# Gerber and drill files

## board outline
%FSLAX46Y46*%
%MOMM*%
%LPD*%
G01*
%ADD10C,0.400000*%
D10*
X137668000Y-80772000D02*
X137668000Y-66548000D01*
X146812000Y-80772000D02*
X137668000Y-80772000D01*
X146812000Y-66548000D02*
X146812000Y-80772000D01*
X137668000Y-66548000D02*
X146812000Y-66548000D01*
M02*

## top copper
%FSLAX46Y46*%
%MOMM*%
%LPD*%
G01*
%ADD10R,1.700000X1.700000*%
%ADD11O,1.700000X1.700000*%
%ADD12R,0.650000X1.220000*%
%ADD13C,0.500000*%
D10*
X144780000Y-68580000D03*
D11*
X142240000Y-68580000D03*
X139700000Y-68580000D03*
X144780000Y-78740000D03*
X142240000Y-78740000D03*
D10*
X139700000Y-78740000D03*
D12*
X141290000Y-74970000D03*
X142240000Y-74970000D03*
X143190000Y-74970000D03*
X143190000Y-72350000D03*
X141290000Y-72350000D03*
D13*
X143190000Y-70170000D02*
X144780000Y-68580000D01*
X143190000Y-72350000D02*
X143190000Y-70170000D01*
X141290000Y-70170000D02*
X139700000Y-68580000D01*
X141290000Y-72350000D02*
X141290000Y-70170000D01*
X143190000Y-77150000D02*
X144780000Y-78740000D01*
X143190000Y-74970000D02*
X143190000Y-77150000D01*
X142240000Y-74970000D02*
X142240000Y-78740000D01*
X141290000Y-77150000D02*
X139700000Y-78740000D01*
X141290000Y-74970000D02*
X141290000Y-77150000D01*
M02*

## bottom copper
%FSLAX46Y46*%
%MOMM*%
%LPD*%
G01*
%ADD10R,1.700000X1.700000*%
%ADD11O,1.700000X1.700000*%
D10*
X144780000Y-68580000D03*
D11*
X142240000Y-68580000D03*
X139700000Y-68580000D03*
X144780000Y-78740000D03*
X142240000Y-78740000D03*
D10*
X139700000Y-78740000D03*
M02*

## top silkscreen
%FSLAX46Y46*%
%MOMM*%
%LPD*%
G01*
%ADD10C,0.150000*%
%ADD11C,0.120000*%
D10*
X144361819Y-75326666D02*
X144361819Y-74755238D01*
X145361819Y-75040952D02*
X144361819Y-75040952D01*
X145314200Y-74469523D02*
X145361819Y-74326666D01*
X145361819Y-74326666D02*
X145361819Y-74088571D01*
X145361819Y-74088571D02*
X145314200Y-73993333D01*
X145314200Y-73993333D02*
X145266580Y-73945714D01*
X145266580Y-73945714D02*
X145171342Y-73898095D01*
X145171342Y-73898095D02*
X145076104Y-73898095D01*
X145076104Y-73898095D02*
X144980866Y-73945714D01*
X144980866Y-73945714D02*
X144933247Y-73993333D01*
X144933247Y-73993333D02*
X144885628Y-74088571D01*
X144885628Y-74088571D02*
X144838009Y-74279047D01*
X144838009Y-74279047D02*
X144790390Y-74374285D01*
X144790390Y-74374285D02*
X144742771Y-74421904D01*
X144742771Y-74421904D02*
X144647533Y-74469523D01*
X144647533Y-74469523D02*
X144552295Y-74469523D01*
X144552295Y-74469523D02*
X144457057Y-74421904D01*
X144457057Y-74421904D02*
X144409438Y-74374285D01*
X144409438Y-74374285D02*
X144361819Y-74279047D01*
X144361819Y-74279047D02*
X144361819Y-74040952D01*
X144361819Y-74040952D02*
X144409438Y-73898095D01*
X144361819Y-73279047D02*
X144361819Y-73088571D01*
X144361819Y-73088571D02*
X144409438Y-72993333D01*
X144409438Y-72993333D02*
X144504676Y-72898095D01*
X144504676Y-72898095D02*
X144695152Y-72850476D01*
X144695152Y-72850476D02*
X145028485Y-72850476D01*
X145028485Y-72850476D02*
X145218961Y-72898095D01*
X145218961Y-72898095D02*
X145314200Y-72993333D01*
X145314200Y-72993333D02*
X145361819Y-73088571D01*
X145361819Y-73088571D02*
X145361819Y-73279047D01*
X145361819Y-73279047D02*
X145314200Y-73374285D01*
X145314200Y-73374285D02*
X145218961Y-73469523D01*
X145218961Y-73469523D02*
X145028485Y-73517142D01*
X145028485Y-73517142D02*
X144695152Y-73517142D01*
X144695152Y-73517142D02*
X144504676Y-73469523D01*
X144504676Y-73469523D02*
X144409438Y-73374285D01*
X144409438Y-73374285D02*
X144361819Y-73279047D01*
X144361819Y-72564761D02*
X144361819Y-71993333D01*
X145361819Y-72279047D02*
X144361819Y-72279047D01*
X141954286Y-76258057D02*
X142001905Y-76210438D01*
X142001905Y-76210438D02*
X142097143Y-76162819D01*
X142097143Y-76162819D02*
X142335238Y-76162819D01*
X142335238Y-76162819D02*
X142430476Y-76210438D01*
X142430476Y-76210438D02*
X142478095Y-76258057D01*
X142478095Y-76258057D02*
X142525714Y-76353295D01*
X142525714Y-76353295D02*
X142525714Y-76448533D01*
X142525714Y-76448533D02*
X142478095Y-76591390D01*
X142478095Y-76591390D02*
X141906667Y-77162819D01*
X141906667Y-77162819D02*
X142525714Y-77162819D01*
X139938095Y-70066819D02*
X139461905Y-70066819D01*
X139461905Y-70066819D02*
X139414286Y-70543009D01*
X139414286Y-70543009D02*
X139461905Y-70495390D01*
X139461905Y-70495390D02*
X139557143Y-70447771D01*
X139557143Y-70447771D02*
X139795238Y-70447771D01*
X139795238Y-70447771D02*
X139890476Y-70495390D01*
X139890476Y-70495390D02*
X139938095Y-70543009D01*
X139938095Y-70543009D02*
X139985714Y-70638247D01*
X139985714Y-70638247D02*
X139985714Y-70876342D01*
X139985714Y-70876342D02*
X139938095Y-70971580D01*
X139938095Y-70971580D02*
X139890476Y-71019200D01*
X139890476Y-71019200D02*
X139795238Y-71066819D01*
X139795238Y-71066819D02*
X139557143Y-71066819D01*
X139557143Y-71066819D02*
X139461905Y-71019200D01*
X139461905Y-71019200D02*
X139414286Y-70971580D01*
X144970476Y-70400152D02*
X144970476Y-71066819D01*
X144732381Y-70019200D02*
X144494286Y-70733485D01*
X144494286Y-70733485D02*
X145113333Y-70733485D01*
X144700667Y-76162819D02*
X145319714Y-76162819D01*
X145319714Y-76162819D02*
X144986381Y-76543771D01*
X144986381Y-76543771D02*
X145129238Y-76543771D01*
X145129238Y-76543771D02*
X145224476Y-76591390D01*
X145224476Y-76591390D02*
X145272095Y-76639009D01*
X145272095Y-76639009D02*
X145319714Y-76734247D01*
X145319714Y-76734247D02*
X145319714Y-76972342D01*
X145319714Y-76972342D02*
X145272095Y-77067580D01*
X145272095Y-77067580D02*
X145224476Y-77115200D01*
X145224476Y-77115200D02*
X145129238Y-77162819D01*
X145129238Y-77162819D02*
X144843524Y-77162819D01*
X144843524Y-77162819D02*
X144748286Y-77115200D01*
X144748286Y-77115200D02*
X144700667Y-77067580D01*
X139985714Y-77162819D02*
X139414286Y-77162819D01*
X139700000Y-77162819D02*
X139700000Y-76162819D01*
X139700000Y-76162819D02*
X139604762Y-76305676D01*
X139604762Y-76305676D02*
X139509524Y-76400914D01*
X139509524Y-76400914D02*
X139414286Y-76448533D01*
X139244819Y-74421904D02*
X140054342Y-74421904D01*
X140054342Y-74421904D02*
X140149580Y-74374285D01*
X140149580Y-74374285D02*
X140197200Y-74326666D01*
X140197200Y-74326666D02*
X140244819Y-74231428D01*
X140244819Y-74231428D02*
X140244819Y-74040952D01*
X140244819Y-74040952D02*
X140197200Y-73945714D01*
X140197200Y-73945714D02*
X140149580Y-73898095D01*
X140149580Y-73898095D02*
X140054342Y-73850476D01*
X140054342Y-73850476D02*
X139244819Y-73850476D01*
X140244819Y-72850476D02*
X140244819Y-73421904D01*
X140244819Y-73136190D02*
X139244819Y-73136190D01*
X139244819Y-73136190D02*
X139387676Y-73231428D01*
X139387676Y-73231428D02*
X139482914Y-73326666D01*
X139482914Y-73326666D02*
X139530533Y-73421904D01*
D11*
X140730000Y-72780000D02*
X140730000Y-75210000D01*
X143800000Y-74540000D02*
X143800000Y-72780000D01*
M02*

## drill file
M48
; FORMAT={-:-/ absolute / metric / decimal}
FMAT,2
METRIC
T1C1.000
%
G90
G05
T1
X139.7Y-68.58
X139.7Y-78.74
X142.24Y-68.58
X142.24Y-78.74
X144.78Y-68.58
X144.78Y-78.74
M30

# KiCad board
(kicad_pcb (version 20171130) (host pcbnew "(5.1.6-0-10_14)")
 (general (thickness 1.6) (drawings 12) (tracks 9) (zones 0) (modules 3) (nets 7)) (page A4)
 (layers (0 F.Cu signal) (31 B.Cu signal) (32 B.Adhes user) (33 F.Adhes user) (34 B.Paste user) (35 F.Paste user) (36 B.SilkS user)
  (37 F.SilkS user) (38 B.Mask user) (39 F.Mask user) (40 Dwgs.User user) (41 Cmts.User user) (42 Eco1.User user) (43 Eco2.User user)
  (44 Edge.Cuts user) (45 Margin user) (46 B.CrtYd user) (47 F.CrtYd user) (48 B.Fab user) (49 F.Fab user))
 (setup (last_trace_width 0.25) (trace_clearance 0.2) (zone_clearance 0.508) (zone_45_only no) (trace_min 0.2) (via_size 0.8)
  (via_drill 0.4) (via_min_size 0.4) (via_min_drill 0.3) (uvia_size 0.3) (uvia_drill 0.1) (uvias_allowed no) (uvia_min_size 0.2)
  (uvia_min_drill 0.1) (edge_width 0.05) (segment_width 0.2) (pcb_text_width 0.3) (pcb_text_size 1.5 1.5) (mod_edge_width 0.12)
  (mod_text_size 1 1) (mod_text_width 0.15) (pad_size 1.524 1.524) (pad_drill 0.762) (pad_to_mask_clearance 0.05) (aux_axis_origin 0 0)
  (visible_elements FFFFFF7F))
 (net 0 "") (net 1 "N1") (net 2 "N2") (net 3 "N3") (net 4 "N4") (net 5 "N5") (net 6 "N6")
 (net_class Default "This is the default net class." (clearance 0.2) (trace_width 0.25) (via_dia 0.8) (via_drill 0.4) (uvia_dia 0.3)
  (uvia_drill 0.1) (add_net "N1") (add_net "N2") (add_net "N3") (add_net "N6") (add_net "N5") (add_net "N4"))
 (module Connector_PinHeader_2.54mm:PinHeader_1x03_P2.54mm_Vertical (layer B.Cu) (at 144.78 68.58 90)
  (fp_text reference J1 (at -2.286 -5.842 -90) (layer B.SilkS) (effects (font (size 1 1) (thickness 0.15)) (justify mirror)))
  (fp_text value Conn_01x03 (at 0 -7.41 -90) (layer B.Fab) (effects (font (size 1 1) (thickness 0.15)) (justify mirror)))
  (pad 1 thru_hole rect (at 0 0 90) (size 1.7 1.7) (drill 1) (layers *.Cu *.Mask) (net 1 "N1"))
  (pad 2 thru_hole oval (at 0 -2.54 90) (size 1.7 1.7) (drill 1) (layers *.Cu *.Mask) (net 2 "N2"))
  (pad 3 thru_hole oval (at 0 -5.08 90) (size 1.7 1.7) (drill 1) (layers *.Cu *.Mask) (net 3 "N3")))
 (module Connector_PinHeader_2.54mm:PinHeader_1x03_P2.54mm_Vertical (layer B.Cu) (at 139.7 78.74 270)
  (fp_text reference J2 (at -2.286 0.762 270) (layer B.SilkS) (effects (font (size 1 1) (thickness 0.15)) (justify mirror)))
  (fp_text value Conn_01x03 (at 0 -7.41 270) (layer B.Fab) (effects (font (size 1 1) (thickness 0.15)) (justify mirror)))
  (pad 3 thru_hole oval (at 0 -5.08 270) (size 1.7 1.7) (drill 1) (layers *.Cu *.Mask) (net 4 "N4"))
  (pad 2 thru_hole oval (at 0 -2.54 270) (size 1.7 1.7) (drill 1) (layers *.Cu *.Mask) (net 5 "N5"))
  (pad 1 thru_hole rect (at 0 0 270) (size 1.7 1.7) (drill 1) (layers *.Cu *.Mask) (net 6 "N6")))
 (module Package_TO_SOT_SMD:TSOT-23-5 (layer F.Cu) (at 142.24 73.66 90)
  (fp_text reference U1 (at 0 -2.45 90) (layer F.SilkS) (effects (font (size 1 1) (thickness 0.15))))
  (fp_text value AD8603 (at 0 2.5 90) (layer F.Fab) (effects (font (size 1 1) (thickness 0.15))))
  (fp_line (start 0.88 -1.51) (end -1.55 -1.51) (layer F.SilkS) (width 0.12))
  (fp_line (start -0.88 1.56) (end 0.88 1.56) (layer F.SilkS) (width 0.12))
  (pad 1 smd rect (at -1.31 -0.95 90) (size 1.22 0.65) (layers F.Cu F.Paste F.Mask) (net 6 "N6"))
  (pad 2 smd rect (at -1.31 0 90) (size 1.22 0.65) (layers F.Cu F.Paste F.Mask) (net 5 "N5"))
  (pad 3 smd rect (at -1.31 0.95 90) (size 1.22 0.65) (layers F.Cu F.Paste F.Mask) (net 4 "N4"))
  (pad 4 smd rect (at 1.31 0.95 90) (size 1.22 0.65) (layers F.Cu F.Paste F.Mask) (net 1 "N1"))
  (pad 5 smd rect (at 1.31 -0.95 90) (size 1.22 0.65) (layers F.Cu F.Paste F.Mask) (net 3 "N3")))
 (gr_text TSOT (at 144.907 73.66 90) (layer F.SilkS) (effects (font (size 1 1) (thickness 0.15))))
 (gr_line (start 137.668 80.772) (end 137.668 66.548) (layer Edge.Cuts) (width 0.4))
 (gr_line (start 146.812 80.772) (end 137.668 80.772) (layer Edge.Cuts) (width 0.4))
 (gr_line (start 146.812 66.548) (end 146.812 80.772) (layer Edge.Cuts) (width 0.4))
 (gr_line (start 137.668 66.548) (end 146.812 66.548) (layer Edge.Cuts) (width 0.4))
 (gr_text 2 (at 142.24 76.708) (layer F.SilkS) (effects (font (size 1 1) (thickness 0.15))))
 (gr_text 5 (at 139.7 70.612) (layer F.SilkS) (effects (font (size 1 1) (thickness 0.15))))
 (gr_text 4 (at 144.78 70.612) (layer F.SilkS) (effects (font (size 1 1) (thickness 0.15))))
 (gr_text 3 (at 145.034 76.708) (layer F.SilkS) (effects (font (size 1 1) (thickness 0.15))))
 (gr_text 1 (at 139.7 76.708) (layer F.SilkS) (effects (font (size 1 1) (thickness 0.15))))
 (segment (start 143.19 70.17) (end 144.78 68.58) (width 0.5) (layer F.Cu) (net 1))
 (segment (start 143.19 72.35) (end 143.19 70.17) (width 0.5) (layer F.Cu) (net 1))
 (segment (start 141.29 70.17) (end 139.7 68.58) (width 0.5) (layer F.Cu) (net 3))
 (segment (start 141.29 72.35) (end 141.29 70.17) (width 0.5) (layer F.Cu) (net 3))
 (segment (start 143.19 77.15) (end 144.78 78.74) (width 0.5) (layer F.Cu) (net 4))
 (segment (start 143.19 74.97) (end 143.19 77.15) (width 0.5) (layer F.Cu) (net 4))
 (segment (start 142.24 74.97) (end 142.24 78.74) (width 0.5) (layer F.Cu) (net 5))
 (segment (start 141.29 77.15) (end 139.7 78.74) (width 0.5) (layer F.Cu) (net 6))
 (segment (start 141.29 74.97) (end 141.29 77.15) (width 0.5) (layer F.Cu) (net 6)))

